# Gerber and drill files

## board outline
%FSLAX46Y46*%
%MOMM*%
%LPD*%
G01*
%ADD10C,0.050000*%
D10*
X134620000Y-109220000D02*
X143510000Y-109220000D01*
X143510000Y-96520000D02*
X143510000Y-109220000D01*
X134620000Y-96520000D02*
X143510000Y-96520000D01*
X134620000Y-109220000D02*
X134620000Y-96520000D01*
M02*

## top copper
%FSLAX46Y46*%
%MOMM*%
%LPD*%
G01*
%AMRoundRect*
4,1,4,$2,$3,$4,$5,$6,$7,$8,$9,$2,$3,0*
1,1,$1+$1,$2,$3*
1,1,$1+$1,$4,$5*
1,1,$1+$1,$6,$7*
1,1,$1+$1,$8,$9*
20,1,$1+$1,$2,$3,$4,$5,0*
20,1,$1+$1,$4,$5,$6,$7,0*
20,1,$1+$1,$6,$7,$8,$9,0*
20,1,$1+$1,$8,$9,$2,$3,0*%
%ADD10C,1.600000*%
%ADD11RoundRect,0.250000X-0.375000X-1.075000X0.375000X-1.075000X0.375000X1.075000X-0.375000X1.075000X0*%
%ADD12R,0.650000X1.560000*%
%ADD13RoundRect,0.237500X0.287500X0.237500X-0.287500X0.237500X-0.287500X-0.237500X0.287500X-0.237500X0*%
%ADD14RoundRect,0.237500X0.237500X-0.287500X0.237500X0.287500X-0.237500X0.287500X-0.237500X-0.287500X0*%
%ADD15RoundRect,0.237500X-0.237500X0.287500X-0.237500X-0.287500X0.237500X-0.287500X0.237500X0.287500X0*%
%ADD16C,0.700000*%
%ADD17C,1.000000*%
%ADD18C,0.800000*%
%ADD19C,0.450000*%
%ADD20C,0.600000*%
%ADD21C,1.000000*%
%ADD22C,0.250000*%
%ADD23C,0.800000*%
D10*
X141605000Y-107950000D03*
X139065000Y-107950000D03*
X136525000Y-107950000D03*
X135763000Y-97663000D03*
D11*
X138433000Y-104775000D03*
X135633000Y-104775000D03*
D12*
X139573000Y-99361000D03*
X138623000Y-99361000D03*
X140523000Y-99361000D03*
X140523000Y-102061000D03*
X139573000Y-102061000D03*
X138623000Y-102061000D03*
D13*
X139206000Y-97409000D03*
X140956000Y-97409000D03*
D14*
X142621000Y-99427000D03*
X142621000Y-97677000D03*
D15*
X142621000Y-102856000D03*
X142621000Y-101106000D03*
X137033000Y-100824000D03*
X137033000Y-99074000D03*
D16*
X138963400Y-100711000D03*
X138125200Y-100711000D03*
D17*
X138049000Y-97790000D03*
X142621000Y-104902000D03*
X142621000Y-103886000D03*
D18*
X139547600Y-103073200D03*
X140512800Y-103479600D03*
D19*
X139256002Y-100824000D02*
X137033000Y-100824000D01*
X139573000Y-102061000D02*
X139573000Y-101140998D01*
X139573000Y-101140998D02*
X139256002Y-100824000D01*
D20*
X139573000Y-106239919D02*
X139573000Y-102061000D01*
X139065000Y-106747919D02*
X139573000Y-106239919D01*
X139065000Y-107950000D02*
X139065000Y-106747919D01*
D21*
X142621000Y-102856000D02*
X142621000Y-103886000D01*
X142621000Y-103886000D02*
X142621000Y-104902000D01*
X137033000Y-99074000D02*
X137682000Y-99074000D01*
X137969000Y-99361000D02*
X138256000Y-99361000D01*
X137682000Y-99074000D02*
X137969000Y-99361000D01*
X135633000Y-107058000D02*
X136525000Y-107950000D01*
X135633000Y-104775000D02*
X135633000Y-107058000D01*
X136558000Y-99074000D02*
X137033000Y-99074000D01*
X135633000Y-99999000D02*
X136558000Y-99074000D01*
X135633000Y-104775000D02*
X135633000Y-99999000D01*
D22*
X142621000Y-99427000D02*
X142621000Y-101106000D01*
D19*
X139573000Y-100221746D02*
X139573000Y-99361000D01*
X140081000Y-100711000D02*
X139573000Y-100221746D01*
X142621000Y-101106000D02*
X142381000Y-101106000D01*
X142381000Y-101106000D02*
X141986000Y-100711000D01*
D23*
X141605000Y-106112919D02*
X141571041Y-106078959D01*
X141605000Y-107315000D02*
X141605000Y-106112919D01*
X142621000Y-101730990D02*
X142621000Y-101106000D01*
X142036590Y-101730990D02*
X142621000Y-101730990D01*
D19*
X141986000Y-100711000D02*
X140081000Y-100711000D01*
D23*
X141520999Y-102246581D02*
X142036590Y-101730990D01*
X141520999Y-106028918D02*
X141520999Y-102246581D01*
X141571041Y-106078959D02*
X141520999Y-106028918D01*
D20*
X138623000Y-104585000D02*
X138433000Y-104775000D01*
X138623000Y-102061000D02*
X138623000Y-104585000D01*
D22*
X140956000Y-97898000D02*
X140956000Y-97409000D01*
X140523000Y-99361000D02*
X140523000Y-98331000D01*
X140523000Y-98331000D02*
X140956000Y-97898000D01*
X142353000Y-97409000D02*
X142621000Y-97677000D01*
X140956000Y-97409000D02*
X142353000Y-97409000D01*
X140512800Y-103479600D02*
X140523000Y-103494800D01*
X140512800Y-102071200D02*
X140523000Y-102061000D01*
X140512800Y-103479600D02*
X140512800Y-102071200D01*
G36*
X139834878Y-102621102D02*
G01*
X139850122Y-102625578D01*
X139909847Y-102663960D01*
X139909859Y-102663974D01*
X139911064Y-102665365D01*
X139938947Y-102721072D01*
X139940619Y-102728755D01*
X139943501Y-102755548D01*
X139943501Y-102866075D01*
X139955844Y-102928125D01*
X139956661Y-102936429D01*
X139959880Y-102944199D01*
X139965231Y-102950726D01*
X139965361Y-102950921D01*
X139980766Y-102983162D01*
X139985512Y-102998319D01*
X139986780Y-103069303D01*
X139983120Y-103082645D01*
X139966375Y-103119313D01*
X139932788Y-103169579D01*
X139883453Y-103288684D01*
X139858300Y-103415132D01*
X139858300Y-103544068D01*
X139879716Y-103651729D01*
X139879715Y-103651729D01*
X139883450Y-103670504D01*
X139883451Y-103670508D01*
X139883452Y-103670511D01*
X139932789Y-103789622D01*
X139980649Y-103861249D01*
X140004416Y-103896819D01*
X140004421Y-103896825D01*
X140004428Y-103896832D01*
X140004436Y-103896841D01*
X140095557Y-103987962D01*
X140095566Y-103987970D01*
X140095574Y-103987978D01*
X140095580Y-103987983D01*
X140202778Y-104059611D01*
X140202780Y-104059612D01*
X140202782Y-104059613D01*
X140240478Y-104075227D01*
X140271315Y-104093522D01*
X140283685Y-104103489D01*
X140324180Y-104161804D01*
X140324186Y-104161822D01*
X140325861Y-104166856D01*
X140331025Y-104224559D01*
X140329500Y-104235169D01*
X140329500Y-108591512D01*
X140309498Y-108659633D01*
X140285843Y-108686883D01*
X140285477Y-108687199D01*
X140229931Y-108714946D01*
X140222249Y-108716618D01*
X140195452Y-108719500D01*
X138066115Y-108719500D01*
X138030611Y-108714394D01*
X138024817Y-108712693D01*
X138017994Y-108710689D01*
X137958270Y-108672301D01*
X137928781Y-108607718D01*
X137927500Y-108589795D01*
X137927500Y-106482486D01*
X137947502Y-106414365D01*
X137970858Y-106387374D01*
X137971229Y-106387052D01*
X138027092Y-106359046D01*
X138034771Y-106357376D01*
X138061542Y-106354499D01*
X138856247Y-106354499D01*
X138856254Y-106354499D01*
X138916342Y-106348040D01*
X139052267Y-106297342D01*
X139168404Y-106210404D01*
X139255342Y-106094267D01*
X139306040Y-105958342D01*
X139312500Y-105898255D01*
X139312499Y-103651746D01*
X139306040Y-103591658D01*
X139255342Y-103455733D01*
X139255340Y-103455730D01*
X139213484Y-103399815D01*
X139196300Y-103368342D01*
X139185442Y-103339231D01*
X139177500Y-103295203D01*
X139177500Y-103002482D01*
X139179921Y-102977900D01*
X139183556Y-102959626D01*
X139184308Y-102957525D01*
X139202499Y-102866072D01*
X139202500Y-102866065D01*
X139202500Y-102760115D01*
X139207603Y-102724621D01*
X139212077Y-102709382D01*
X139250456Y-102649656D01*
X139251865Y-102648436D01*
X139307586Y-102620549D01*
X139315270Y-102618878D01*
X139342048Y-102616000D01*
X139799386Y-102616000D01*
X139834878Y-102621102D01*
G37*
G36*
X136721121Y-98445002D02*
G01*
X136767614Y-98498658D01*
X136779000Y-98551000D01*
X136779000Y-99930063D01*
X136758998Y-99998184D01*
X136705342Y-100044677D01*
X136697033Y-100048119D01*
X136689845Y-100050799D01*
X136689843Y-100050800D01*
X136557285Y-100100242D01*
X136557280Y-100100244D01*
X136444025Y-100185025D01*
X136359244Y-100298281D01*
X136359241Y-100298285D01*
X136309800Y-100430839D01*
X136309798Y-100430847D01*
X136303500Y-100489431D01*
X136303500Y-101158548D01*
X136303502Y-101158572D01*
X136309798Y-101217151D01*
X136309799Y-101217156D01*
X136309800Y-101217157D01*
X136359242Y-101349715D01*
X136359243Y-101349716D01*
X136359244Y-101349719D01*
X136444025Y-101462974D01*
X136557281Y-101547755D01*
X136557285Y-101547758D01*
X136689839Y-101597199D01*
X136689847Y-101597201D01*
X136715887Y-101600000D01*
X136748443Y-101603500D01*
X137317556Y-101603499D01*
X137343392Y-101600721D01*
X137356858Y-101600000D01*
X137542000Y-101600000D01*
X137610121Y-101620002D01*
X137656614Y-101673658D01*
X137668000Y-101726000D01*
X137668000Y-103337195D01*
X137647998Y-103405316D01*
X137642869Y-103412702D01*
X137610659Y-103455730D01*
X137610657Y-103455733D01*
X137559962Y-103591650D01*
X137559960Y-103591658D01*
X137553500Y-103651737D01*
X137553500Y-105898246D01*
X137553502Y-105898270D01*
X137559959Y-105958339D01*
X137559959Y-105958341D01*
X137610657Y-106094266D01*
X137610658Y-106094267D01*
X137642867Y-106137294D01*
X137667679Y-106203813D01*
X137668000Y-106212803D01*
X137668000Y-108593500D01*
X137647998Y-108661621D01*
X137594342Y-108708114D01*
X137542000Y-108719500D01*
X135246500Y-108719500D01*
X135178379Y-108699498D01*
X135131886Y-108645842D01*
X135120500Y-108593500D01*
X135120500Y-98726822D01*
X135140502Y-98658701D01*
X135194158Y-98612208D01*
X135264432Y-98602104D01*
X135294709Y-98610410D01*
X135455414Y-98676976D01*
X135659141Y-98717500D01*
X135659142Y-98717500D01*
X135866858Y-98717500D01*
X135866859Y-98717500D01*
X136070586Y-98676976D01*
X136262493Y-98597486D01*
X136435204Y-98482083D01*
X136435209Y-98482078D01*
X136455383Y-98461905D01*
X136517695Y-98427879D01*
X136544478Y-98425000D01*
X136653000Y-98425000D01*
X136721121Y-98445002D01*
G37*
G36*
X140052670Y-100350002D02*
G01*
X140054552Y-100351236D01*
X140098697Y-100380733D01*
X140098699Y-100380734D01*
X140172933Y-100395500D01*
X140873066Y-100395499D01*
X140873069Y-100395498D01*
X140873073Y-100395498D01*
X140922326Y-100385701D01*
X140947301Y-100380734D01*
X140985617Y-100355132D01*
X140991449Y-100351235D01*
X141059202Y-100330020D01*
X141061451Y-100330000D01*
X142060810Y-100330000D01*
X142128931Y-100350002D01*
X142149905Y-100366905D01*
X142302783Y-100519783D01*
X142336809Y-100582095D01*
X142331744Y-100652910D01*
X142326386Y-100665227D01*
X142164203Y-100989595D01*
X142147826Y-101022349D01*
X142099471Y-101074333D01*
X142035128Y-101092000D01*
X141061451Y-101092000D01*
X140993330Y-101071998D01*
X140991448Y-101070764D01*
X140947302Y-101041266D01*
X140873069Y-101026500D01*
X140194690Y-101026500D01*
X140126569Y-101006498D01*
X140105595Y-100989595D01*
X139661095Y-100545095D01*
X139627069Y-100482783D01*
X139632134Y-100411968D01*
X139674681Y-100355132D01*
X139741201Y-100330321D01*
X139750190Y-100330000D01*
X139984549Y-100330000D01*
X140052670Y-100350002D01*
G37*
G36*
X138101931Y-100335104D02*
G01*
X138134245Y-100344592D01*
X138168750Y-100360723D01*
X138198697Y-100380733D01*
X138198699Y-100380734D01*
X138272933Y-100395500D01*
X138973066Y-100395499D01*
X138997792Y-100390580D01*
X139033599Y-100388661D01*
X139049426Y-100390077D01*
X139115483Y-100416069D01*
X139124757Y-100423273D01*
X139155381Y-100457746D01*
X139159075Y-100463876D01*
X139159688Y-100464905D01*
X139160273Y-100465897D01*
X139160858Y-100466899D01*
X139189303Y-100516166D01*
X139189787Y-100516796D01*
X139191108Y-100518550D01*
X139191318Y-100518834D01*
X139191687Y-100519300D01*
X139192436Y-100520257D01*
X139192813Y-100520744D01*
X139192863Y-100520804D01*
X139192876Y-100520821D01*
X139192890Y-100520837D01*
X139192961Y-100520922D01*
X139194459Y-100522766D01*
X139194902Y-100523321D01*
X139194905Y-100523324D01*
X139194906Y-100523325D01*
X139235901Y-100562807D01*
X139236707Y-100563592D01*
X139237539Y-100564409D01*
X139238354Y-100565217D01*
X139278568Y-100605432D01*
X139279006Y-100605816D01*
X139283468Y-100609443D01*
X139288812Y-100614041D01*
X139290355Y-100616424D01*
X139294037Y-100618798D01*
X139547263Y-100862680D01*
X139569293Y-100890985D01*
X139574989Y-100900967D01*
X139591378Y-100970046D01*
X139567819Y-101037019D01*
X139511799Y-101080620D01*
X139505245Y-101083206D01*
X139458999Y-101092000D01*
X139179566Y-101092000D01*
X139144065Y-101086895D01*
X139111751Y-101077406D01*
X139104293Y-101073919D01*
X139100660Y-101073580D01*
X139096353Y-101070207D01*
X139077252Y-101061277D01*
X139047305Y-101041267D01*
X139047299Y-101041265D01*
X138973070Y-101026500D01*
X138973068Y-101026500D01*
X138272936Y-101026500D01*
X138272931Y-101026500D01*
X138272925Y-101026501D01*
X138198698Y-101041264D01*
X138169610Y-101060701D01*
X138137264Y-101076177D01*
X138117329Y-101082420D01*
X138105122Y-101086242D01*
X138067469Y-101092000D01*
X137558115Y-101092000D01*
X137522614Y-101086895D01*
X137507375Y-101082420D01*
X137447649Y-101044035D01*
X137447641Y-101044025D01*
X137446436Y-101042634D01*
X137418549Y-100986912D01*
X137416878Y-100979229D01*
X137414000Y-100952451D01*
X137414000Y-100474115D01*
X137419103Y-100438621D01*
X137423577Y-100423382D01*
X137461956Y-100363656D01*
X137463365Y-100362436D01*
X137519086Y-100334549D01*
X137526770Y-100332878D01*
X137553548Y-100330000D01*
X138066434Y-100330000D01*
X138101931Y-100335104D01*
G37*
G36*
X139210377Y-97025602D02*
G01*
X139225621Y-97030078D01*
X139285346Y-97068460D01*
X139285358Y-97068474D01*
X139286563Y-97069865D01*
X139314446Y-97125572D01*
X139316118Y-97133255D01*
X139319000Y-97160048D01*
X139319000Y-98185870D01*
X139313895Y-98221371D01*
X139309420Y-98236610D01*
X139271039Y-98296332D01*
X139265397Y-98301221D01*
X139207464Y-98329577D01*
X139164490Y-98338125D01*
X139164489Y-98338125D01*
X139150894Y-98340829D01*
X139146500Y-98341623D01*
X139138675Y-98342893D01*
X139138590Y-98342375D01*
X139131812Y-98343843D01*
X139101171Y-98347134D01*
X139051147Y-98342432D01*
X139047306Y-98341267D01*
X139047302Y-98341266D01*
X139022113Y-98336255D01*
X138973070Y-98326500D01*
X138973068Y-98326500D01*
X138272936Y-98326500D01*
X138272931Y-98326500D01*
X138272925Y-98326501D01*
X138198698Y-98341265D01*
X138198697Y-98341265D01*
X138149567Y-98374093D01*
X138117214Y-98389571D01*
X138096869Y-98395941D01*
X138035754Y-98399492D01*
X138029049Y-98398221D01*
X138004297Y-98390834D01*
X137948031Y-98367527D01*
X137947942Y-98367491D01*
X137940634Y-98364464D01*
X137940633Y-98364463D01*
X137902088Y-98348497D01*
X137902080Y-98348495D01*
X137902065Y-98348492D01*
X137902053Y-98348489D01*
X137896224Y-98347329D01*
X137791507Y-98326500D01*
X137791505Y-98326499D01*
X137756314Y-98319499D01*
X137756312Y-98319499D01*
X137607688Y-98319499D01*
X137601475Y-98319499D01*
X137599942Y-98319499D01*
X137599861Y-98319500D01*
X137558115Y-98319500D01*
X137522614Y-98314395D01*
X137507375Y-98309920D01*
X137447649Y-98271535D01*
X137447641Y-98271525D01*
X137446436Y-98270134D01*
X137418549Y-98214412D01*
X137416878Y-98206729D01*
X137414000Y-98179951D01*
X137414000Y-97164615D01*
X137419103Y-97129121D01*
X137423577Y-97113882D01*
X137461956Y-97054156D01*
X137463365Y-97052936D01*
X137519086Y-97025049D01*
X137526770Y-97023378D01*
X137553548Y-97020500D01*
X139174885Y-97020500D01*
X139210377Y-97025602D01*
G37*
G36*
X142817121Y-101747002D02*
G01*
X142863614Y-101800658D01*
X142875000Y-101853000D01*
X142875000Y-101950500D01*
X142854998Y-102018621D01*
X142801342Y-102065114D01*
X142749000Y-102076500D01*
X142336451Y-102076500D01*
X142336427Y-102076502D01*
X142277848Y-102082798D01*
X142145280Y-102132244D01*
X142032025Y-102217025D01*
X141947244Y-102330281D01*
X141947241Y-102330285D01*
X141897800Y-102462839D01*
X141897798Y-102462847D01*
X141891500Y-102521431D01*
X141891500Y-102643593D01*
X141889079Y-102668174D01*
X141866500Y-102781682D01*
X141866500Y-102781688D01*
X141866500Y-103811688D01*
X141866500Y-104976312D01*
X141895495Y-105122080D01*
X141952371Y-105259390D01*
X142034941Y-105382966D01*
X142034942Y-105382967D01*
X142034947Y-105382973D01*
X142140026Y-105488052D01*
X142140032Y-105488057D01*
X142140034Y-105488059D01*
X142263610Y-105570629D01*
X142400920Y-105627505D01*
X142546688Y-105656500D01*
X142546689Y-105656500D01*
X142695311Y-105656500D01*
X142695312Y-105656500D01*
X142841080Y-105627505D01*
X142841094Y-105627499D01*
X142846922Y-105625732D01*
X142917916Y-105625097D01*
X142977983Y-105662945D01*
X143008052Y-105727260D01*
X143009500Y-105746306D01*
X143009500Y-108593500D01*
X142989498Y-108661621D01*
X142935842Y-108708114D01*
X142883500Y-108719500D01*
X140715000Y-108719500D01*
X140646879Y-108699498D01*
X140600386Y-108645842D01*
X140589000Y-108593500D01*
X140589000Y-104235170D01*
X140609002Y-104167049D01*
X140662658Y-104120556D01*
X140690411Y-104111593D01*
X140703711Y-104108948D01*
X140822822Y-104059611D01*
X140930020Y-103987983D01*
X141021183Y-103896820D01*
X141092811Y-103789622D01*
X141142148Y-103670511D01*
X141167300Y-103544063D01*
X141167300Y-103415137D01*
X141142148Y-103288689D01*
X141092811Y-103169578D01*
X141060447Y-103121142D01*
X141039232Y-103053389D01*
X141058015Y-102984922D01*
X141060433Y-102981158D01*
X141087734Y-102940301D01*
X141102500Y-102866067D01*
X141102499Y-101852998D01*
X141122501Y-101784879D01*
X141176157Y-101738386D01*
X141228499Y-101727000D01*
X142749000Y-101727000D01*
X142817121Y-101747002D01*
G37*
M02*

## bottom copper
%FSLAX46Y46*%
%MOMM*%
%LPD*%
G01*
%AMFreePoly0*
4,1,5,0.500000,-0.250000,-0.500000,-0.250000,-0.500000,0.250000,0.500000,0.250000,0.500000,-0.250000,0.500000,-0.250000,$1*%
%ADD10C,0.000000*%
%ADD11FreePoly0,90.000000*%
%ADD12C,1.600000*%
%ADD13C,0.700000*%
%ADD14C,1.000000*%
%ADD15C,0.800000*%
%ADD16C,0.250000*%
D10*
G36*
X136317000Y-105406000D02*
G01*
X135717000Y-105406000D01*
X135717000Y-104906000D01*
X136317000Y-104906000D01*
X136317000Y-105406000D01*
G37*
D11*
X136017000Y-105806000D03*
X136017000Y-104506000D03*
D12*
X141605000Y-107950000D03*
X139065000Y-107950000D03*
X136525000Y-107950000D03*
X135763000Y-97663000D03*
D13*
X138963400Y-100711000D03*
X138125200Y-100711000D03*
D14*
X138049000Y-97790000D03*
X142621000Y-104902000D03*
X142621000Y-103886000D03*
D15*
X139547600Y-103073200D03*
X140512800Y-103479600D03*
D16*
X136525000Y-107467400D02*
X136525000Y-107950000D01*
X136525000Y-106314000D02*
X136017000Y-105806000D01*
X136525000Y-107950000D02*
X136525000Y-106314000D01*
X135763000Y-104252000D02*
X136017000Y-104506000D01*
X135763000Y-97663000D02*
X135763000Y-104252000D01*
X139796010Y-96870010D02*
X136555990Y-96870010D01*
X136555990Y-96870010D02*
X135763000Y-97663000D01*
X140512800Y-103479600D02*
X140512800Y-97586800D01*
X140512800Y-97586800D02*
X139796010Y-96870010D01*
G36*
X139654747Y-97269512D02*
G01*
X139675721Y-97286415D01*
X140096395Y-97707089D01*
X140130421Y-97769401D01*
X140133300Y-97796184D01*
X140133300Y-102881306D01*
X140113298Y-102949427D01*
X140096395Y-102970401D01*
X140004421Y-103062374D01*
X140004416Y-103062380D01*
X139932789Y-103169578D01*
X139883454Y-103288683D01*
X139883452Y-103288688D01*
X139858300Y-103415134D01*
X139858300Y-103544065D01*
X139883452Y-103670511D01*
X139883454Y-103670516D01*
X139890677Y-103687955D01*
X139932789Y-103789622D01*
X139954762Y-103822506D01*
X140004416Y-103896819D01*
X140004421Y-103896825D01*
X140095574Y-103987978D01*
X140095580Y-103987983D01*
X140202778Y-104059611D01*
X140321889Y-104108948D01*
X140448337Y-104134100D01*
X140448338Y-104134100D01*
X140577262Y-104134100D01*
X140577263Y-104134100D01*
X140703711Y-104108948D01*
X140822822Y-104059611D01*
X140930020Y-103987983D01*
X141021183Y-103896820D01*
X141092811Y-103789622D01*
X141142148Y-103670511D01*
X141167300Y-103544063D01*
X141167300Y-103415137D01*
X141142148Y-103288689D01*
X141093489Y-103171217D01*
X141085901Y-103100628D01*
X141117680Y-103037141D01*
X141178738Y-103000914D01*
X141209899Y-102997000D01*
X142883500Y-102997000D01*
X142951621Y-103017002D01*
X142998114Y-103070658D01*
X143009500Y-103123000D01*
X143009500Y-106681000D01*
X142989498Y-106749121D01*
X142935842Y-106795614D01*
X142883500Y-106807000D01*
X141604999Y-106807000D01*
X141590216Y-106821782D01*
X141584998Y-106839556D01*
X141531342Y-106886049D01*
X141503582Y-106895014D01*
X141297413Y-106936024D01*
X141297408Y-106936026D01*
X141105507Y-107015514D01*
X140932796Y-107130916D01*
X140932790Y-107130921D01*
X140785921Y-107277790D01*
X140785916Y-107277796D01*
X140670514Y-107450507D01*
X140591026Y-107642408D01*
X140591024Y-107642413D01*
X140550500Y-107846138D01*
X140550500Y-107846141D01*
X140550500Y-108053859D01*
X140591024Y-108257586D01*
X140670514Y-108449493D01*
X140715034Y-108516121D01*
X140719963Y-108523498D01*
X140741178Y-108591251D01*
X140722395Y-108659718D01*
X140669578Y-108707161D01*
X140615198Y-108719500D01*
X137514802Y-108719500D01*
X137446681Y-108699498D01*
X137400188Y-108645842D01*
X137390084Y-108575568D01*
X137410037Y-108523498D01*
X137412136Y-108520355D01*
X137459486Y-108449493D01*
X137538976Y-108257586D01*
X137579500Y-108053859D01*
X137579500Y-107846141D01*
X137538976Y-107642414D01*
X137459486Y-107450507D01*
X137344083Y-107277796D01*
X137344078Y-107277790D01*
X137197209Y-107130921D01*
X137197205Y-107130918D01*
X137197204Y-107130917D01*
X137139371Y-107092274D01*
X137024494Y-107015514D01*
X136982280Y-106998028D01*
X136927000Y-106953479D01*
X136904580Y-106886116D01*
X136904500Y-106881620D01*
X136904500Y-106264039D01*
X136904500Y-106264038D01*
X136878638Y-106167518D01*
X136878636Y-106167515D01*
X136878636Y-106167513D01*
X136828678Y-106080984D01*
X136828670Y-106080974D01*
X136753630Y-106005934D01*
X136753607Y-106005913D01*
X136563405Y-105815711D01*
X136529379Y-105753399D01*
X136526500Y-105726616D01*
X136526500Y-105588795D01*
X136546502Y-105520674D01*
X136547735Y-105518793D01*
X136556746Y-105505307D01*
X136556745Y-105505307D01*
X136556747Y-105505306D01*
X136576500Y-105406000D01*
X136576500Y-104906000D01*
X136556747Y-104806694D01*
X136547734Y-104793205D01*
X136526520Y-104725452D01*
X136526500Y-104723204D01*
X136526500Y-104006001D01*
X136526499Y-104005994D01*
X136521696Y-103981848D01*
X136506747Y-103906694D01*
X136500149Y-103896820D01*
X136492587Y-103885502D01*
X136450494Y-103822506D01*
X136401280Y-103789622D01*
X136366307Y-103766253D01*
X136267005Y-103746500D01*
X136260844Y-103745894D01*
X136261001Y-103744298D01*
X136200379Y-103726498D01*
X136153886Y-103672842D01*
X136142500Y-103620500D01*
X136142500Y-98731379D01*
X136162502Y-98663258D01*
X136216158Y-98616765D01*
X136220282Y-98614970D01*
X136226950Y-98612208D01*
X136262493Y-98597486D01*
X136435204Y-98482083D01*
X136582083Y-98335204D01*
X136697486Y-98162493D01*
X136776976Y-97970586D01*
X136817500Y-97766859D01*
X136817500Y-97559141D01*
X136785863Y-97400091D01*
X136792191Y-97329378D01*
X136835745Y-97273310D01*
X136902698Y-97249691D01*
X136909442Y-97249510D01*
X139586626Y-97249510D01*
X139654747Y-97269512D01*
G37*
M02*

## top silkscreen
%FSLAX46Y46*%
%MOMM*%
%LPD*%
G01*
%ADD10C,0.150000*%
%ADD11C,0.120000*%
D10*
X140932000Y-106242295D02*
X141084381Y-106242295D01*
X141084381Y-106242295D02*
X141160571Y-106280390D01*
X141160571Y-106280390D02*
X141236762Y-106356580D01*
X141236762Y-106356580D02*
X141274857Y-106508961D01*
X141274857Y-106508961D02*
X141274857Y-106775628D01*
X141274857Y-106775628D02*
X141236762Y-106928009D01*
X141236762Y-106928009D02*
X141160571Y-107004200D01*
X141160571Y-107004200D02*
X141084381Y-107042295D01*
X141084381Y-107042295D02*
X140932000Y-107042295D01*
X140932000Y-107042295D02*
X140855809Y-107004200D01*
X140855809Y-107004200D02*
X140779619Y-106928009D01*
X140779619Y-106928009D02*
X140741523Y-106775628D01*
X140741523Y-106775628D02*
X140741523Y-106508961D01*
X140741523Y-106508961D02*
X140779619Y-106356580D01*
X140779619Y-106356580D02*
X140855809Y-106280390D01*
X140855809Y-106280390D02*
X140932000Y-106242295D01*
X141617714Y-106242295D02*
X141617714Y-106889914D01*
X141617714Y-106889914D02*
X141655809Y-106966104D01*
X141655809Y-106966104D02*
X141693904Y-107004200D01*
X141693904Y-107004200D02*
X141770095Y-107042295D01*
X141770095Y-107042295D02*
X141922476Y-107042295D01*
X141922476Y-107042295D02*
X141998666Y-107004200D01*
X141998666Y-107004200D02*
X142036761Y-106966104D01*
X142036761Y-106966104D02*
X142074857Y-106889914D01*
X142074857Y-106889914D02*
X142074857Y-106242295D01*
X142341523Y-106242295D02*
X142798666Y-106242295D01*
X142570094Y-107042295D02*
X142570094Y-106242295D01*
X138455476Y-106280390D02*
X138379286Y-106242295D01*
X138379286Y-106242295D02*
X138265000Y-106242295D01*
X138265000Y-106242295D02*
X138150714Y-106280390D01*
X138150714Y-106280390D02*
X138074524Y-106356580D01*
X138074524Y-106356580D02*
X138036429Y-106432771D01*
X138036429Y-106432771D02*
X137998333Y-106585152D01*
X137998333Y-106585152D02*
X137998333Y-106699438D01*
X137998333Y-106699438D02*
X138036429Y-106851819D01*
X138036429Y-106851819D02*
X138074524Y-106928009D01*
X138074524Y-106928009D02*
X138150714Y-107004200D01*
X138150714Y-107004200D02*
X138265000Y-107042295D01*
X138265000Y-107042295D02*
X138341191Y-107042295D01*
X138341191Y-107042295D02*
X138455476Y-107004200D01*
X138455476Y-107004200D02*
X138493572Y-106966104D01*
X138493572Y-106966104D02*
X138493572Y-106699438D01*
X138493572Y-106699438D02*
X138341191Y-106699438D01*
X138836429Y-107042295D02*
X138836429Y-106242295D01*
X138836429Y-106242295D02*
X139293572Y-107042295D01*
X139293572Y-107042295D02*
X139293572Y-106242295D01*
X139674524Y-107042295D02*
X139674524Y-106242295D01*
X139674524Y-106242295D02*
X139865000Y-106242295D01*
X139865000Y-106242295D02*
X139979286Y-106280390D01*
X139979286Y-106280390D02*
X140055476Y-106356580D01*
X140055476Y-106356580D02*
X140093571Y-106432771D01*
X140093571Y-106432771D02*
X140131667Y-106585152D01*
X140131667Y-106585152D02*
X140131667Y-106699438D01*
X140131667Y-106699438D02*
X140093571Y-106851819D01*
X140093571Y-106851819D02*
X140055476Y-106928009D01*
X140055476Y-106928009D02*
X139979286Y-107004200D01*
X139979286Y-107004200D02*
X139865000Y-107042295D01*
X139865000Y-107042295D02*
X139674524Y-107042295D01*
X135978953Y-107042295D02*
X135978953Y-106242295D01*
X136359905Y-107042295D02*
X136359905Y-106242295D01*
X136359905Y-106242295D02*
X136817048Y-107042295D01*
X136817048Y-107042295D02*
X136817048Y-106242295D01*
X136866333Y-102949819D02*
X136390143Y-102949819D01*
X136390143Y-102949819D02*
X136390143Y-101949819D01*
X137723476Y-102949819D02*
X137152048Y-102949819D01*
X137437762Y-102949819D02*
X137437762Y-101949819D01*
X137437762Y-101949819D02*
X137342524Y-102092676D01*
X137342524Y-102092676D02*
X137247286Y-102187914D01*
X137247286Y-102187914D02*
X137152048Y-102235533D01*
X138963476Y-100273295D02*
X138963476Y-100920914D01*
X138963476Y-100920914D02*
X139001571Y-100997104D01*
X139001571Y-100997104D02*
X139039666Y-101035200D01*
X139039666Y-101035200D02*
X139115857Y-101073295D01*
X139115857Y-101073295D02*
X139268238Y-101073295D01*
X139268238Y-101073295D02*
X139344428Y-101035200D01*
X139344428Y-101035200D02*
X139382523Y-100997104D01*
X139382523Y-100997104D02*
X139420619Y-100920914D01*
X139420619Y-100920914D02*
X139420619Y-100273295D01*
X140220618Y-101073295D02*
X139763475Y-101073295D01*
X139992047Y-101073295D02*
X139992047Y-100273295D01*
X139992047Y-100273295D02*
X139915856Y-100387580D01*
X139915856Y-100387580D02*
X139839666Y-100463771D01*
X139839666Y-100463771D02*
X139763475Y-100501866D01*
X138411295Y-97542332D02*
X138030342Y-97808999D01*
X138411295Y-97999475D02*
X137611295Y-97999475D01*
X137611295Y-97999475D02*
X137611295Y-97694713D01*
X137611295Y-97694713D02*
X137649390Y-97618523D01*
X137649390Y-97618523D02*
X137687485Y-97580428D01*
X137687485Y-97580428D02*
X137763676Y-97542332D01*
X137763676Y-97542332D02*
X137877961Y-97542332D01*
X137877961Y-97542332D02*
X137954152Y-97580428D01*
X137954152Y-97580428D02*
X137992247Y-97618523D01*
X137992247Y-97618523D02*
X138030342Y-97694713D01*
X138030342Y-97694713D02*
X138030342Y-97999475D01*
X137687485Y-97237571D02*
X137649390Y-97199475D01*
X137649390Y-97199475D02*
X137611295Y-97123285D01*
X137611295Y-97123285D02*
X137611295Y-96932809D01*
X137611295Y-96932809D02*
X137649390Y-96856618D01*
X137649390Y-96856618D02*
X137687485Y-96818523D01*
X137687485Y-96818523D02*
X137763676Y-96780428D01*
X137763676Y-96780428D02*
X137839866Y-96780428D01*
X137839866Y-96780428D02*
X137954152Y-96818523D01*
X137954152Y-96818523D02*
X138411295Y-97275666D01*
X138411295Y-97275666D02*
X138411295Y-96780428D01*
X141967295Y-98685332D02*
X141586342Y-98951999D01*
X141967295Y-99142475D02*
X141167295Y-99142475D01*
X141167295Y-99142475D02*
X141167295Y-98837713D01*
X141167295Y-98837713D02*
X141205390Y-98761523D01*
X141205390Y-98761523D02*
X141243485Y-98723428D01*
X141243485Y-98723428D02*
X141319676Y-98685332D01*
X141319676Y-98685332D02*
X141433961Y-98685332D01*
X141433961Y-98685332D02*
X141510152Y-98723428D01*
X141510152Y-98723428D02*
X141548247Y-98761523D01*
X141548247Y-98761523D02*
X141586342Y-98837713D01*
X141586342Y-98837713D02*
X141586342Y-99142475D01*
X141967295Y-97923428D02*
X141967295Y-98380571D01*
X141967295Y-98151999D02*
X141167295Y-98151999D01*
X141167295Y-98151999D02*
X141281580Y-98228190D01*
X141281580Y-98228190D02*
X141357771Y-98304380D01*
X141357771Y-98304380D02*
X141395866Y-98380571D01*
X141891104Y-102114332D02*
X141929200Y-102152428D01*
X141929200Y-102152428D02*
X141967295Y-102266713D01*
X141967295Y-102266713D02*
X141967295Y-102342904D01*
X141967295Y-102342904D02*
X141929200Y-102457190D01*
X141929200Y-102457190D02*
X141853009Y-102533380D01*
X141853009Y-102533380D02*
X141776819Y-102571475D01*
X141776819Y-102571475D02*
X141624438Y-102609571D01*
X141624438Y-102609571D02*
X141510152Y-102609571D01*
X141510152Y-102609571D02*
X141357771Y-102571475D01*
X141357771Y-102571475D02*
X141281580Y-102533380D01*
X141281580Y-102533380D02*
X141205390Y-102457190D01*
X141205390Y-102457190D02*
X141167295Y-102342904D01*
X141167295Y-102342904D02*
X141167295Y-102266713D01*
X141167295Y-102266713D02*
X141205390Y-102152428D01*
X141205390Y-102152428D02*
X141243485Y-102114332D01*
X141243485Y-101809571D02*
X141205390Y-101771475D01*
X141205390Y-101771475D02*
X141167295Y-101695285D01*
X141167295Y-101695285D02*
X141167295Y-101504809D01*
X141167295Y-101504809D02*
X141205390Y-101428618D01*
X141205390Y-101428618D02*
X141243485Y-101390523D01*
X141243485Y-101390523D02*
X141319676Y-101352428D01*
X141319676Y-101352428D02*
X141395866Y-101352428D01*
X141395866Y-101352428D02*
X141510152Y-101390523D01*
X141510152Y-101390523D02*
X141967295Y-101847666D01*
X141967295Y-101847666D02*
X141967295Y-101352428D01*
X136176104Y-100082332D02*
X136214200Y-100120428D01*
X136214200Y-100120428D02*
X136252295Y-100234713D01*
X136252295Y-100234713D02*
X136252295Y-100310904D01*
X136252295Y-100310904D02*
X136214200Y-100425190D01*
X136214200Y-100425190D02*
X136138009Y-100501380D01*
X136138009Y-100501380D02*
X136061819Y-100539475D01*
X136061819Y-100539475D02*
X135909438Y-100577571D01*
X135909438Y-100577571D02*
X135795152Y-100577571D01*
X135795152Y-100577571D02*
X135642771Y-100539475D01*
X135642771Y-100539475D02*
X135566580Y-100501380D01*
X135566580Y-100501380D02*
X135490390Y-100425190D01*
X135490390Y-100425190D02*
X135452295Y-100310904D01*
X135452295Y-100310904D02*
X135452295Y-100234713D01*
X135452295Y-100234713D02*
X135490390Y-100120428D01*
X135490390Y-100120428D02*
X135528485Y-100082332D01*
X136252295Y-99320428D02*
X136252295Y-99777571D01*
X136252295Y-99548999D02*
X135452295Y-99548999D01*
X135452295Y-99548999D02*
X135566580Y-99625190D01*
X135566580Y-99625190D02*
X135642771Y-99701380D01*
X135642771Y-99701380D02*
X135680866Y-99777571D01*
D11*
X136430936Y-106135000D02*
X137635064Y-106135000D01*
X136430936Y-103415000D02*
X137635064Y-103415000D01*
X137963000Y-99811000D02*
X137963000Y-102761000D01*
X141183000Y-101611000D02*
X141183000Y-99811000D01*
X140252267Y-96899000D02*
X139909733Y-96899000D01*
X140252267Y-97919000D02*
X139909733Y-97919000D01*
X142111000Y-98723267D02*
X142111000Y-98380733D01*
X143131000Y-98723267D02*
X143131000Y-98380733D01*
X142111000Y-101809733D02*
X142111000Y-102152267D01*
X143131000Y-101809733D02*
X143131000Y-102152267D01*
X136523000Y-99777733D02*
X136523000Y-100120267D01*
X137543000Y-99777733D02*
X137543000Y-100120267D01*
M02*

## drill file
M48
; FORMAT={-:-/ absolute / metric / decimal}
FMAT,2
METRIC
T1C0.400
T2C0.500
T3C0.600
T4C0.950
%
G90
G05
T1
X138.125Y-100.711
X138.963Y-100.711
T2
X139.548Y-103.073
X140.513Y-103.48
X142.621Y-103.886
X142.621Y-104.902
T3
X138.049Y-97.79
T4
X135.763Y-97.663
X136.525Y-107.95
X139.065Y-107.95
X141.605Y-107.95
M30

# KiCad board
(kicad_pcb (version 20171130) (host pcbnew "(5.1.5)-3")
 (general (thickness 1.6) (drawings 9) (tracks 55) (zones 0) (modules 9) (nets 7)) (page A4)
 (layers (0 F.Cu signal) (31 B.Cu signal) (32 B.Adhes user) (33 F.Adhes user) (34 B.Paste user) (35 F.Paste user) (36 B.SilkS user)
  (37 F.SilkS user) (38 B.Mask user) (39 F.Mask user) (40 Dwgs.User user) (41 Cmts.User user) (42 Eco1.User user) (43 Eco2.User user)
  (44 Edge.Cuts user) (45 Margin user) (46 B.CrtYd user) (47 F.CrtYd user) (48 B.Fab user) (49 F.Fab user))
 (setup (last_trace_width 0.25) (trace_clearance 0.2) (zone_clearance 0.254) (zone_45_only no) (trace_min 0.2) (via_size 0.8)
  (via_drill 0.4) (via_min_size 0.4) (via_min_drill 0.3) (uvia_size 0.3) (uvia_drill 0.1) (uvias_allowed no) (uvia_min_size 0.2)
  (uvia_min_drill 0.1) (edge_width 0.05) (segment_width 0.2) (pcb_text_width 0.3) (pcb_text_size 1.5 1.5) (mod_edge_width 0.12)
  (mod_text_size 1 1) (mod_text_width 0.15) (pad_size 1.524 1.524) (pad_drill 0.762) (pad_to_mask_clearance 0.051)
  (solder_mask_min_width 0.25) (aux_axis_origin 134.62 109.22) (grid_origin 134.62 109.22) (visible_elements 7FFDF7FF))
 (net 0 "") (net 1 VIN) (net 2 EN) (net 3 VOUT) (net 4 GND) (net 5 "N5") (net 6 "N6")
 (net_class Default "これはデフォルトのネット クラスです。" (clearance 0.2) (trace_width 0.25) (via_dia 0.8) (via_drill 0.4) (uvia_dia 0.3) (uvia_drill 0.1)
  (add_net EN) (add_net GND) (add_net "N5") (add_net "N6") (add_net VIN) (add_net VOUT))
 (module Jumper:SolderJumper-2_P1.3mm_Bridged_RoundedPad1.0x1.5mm (layer B.Cu) (at 136.017 105.156 90)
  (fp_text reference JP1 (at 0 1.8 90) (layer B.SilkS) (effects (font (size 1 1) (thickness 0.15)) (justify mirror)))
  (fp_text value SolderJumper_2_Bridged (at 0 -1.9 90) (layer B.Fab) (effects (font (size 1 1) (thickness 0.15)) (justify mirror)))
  (fp_poly (pts (xy 0.25 0.3) (xy -0.25 0.3) (xy -0.25 -0.3) (xy 0.25 -0.3)) (layer B.Cu) (width 0))
  (pad 1 smd custom (at -0.65 0 90) (size 1 0.5) (layers B.Cu B.Mask) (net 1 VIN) (zone_connect 2)
   (options (clearance outline) (anchor rect)) (primitives))
  (pad 2 smd custom (at 0.65 0 90) (size 1 0.5) (layers B.Cu B.Mask) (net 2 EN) (zone_connect 2) (options (clearance outline) (anchor rect))
   (primitives)))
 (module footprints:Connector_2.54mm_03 (layer F.Cu) (at 136.525 107.95 90)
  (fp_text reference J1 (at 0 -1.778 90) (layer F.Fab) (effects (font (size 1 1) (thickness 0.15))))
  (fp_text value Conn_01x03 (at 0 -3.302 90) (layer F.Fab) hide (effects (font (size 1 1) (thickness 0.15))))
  (pad 3 thru_hole circle (at 0 5.08 90) (size 1.6 1.6) (drill 0.95) (layers *.Cu *.Mask) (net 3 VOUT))
  (pad 2 thru_hole circle (at 0 2.54 90) (size 1.6 1.6) (drill 0.95) (layers *.Cu *.Mask) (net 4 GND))
  (pad 1 thru_hole circle (at 0 0 90) (size 1.6 1.6) (drill 0.95) (layers *.Cu *.Mask) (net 1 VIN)))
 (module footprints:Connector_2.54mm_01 (layer F.Cu) (at 135.763 97.663)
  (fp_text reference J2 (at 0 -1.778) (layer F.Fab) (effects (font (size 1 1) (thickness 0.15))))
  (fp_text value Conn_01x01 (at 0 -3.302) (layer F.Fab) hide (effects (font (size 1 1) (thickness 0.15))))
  (pad 1 thru_hole circle (at 0 0) (size 1.6 1.6) (drill 0.95) (layers *.Cu *.Mask) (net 2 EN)))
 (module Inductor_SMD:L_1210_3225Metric (layer F.Cu) (at 137.033 104.775)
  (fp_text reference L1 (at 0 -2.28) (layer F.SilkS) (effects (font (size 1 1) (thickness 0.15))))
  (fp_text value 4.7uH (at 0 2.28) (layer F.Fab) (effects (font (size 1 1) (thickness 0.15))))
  (fp_line (start -0.602064 1.36) (end 0.602064 1.36) (layer F.SilkS) (width 0.12))
  (fp_line (start -0.602064 -1.36) (end 0.602064 -1.36) (layer F.SilkS) (width 0.12))
  (pad 2 smd roundrect (at 1.4 0) (size 1.25 2.65) (layers F.Cu F.Paste F.Mask) (roundrect_rratio 0.2) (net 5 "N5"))
  (pad 1 smd roundrect (at -1.4 0) (size 1.25 2.65) (layers F.Cu F.Paste F.Mask) (roundrect_rratio 0.2) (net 1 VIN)))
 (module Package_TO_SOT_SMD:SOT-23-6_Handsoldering (layer F.Cu) (at 139.573 100.711 90)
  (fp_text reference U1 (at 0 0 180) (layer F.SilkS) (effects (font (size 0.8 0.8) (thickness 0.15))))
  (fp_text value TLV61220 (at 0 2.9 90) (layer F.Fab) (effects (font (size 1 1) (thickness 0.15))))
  (fp_line (start 0.9 -1.61) (end -2.05 -1.61) (layer F.SilkS) (width 0.12))
  (fp_line (start -0.9 1.61) (end 0.9 1.61) (layer F.SilkS) (width 0.12))
  (pad 5 smd rect (at 1.35 0 90) (size 1.56 0.65) (layers F.Cu F.Paste F.Mask) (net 3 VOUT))
  (pad 6 smd rect (at 1.35 -0.95 90) (size 1.56 0.65) (layers F.Cu F.Paste F.Mask) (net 1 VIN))
  (pad 4 smd rect (at 1.35 0.95 90) (size 1.56 0.65) (layers F.Cu F.Paste F.Mask) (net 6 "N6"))
  (pad 3 smd rect (at -1.35 0.95 90) (size 1.56 0.65) (layers F.Cu F.Paste F.Mask) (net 2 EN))
  (pad 2 smd rect (at -1.35 0 90) (size 1.56 0.65) (layers F.Cu F.Paste F.Mask) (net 4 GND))
  (pad 1 smd rect (at -1.35 -0.95 90) (size 1.56 0.65) (layers F.Cu F.Paste F.Mask) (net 5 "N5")))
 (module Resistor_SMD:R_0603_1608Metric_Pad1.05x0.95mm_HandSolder (layer F.Cu) (at 140.081 97.409 180)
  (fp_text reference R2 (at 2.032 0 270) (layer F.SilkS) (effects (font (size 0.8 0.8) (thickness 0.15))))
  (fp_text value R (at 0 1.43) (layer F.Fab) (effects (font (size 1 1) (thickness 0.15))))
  (fp_line (start -0.171267 0.51) (end 0.171267 0.51) (layer F.SilkS) (width 0.12))
  (fp_line (start -0.171267 -0.51) (end 0.171267 -0.51) (layer F.SilkS) (width 0.12))
  (pad 2 smd roundrect (at 0.875 0 180) (size 1.05 0.95) (layers F.Cu F.Paste F.Mask) (roundrect_rratio 0.25) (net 4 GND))
  (pad 1 smd roundrect (at -0.875 0 180) (size 1.05 0.95) (layers F.Cu F.Paste F.Mask) (roundrect_rratio 0.25) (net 6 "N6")))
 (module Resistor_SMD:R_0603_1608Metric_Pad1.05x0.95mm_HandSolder (layer F.Cu) (at 142.621 98.552 90)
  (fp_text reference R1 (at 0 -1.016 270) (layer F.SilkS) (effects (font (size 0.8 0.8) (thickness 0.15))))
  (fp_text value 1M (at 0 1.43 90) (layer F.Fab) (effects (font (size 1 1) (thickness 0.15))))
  (fp_line (start -0.171267 -0.51) (end 0.171267 -0.51) (layer F.SilkS) (width 0.12))
  (fp_line (start -0.171267 0.51) (end 0.171267 0.51) (layer F.SilkS) (width 0.12))
  (pad 1 smd roundrect (at -0.875 0 90) (size 1.05 0.95) (layers F.Cu F.Paste F.Mask) (roundrect_rratio 0.25) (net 3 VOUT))
  (pad 2 smd roundrect (at 0.875 0 90) (size 1.05 0.95) (layers F.Cu F.Paste F.Mask) (roundrect_rratio 0.25) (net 6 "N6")))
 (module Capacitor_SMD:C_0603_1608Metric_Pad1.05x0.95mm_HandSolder (layer F.Cu) (at 142.621 101.981 270)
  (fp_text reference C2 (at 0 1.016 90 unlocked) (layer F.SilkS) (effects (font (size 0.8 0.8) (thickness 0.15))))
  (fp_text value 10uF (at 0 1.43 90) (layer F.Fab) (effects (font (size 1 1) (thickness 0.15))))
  (fp_line (start -0.171267 0.51) (end 0.171267 0.51) (layer F.SilkS) (width 0.12))
  (fp_line (start -0.171267 -0.51) (end 0.171267 -0.51) (layer F.SilkS) (width 0.12))
  (pad 2 smd roundrect (at 0.875 0 270) (size 1.05 0.95) (layers F.Cu F.Paste F.Mask) (roundrect_rratio 0.25) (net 4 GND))
  (pad 1 smd roundrect (at -0.875 0 270) (size 1.05 0.95) (layers F.Cu F.Paste F.Mask) (roundrect_rratio 0.25) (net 3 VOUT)))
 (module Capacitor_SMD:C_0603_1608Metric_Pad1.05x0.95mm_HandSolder (layer F.Cu) (at 137.033 99.949 270)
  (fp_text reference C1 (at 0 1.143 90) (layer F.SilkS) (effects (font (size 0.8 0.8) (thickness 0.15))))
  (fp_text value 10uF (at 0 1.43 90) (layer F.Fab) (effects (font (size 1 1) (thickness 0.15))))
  (fp_line (start -0.171267 0.51) (end 0.171267 0.51) (layer F.SilkS) (width 0.12))
  (fp_line (start -0.171267 -0.51) (end 0.171267 -0.51) (layer F.SilkS) (width 0.12))
  (pad 2 smd roundrect (at 0.875 0 270) (size 1.05 0.95) (layers F.Cu F.Paste F.Mask) (roundrect_rratio 0.25) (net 4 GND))
  (pad 1 smd roundrect (at -0.875 0 270) (size 1.05 0.95) (layers F.Cu F.Paste F.Mask) (roundrect_rratio 0.25) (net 1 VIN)))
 (gr_line (start 134.62 109.22) (end 143.51 109.22) (layer Edge.Cuts) (width 0.05))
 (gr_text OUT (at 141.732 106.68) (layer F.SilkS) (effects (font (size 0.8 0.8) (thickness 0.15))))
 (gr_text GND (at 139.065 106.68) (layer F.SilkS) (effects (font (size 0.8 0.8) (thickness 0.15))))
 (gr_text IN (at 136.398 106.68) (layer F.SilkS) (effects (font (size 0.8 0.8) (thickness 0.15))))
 (gr_line (start 143.51 96.52) (end 143.51 109.22) (layer Edge.Cuts) (width 0.05))
 (gr_line (start 134.62 96.52) (end 143.51 96.52) (layer Edge.Cuts) (width 0.05))
 (gr_line (start 134.62 109.22) (end 134.62 96.52) (layer Edge.Cuts) (width 0.05))
 (via (at 138.9634 100.711) (size 0.7) (drill 0.4) (layers F.Cu B.Cu) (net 4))
 (via (at 138.1252 100.711) (size 0.7) (drill 0.4) (layers F.Cu B.Cu) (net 4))
 (via (at 138.049 97.79) (size 1) (drill 0.6) (layers F.Cu B.Cu) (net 4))
 (segment (start 139.256002 100.824) (end 137.033 100.824) (width 0.45) (layer F.Cu) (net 4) (status 20))
 (segment (start 139.573 102.061) (end 139.573 101.140998) (width 0.45) (layer F.Cu) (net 4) (status 10))
 (segment (start 139.573 101.140998) (end 139.256002 100.824) (width 0.45) (layer F.Cu) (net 4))
 (via (at 142.621 104.902) (size 1) (drill 0.5) (layers F.Cu B.Cu) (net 4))
 (via (at 142.621 103.886) (size 1) (drill 0.5) (layers F.Cu B.Cu) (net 4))
 (segment (start 139.573 106.239919) (end 139.573 102.061) (width 0.6) (layer F.Cu) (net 4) (status 20))
 (segment (start 139.065 106.747919) (end 139.573 106.239919) (width 0.6) (layer F.Cu) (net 4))
 (segment (start 139.065 107.95) (end 139.065 106.747919) (width 0.6) (layer F.Cu) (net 4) (status 10))
 (segment (start 142.621 102.856) (end 142.621 103.886) (width 1) (layer F.Cu) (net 4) (status 10))
 (segment (start 142.621 103.886) (end 142.621 104.902) (width 1) (layer F.Cu) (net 4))
 (via (at 139.5476 103.0732) (size 0.8) (drill 0.5) (layers F.Cu B.Cu) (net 4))
 (segment (start 137.033 99.074) (end 137.682 99.074) (width 1) (layer F.Cu) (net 1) (status 10))
 (segment (start 137.969 99.361) (end 138.256 99.361) (width 1) (layer F.Cu) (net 1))
 (segment (start 137.682 99.074) (end 137.969 99.361) (width 1) (layer F.Cu) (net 1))
 (segment (start 135.633 107.058) (end 136.525 107.95) (width 1) (layer F.Cu) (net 1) (status 20))
 (segment (start 135.633 104.775) (end 135.633 107.058) (width 1) (layer F.Cu) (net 1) (status 10))
 (segment (start 136.558 99.074) (end 137.033 99.074) (width 1) (layer F.Cu) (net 1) (status 30))
 (segment (start 135.633 99.999) (end 136.558 99.074) (width 1) (layer F.Cu) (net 1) (status 20))
 (segment (start 135.633 104.775) (end 135.633 99.999) (width 1) (layer F.Cu) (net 1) (status 10))
 (segment (start 136.525 107.4674) (end 136.525 107.95) (width 0.25) (layer B.Cu) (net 1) (status 30))
 (segment (start 136.525 106.314) (end 136.017 105.806) (width 0.25) (layer B.Cu) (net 1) (status 20))
 (segment (start 136.525 107.95) (end 136.525 106.314) (width 0.25) (layer B.Cu) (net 1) (status 10))
 (segment (start 142.621 99.427) (end 142.621 101.106) (width 0.25) (layer F.Cu) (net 3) (status 30))
 (segment (start 139.573 100.221746) (end 139.573 99.361) (width 0.45) (layer F.Cu) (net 3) (status 20))
 (segment (start 140.081 100.711) (end 139.573 100.221746) (width 0.45) (layer F.Cu) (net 3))
 (segment (start 142.621 101.106) (end 142.381 101.106) (width 0.45) (layer F.Cu) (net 3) (status 30))
 (segment (start 142.381 101.106) (end 141.986 100.711) (width 0.45) (layer F.Cu) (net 3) (status 10))
 (segment (start 141.605 106.112919) (end 141.571041 106.078959) (width 0.8) (layer F.Cu) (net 3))
 (segment (start 141.605 107.315) (end 141.605 106.112919) (width 0.8) (layer F.Cu) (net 3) (status 10))
 (segment (start 142.621 101.73099) (end 142.621 101.106) (width 0.8) (layer F.Cu) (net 3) (status 20))
 (segment (start 142.03659 101.73099) (end 142.621 101.73099) (width 0.8) (layer F.Cu) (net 3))
 (segment (start 141.986 100.711) (end 140.081 100.711) (width 0.45) (layer F.Cu) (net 3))
 (segment (start 141.520999 102.246581) (end 142.03659 101.73099) (width 0.8) (layer F.Cu) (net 3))
 (segment (start 141.520999 106.028918) (end 141.520999 102.246581) (width 0.8) (layer F.Cu) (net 3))
 (segment (start 141.571041 106.078959) (end 141.520999 106.028918) (width 0.8) (layer F.Cu) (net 3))
 (segment (start 138.623 104.585) (end 138.433 104.775) (width 0.6) (layer F.Cu) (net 5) (status 30))
 (segment (start 138.623 102.061) (end 138.623 104.585) (width 0.6) (layer F.Cu) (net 5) (status 30))
 (segment (start 140.956 97.898) (end 140.956 97.409) (width 0.25) (layer F.Cu) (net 6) (status 20))
 (segment (start 140.523 99.361) (end 140.523 98.331) (width 0.25) (layer F.Cu) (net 6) (status 10))
 (segment (start 140.523 98.331) (end 140.956 97.898) (width 0.25) (layer F.Cu) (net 6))
 (segment (start 142.353 97.409) (end 142.621 97.677) (width 0.25) (layer F.Cu) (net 6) (status 30))
 (segment (start 140.956 97.409) (end 142.353 97.409) (width 0.25) (layer F.Cu) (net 6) (status 30))
 (via (at 140.5128 103.4796) (size 0.8) (drill 0.5) (layers F.Cu B.Cu) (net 2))
 (segment (start 140.5128 103.4796) (end 140.523 103.4948) (width 0.25) (layer F.Cu) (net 2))
 (segment (start 140.5128 102.0712) (end 140.523 102.061) (width 0.25) (layer F.Cu) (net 2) (status 30))
 (segment (start 140.5128 103.4796) (end 140.5128 102.0712) (width 0.25) (layer F.Cu) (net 2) (status 20))
 (segment (start 135.763 104.252) (end 136.017 104.506) (width 0.25) (layer B.Cu) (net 2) (status 30))
 (segment (start 135.763 97.663) (end 135.763 104.252) (width 0.25) (layer B.Cu) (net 2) (status 30))
 (segment (start 139.79601 96.87001) (end 136.55599 96.87001) (width 0.25) (layer B.Cu) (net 2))
 (segment (start 136.55599 96.87001) (end 135.763 97.663) (width 0.25) (layer B.Cu) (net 2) (status 20))
 (segment (start 140.5128 103.4796) (end 140.5128 97.5868) (width 0.25) (layer B.Cu) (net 2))
 (segment (start 140.5128 97.5868) (end 139.79601 96.87001) (width 0.25) (layer B.Cu) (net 2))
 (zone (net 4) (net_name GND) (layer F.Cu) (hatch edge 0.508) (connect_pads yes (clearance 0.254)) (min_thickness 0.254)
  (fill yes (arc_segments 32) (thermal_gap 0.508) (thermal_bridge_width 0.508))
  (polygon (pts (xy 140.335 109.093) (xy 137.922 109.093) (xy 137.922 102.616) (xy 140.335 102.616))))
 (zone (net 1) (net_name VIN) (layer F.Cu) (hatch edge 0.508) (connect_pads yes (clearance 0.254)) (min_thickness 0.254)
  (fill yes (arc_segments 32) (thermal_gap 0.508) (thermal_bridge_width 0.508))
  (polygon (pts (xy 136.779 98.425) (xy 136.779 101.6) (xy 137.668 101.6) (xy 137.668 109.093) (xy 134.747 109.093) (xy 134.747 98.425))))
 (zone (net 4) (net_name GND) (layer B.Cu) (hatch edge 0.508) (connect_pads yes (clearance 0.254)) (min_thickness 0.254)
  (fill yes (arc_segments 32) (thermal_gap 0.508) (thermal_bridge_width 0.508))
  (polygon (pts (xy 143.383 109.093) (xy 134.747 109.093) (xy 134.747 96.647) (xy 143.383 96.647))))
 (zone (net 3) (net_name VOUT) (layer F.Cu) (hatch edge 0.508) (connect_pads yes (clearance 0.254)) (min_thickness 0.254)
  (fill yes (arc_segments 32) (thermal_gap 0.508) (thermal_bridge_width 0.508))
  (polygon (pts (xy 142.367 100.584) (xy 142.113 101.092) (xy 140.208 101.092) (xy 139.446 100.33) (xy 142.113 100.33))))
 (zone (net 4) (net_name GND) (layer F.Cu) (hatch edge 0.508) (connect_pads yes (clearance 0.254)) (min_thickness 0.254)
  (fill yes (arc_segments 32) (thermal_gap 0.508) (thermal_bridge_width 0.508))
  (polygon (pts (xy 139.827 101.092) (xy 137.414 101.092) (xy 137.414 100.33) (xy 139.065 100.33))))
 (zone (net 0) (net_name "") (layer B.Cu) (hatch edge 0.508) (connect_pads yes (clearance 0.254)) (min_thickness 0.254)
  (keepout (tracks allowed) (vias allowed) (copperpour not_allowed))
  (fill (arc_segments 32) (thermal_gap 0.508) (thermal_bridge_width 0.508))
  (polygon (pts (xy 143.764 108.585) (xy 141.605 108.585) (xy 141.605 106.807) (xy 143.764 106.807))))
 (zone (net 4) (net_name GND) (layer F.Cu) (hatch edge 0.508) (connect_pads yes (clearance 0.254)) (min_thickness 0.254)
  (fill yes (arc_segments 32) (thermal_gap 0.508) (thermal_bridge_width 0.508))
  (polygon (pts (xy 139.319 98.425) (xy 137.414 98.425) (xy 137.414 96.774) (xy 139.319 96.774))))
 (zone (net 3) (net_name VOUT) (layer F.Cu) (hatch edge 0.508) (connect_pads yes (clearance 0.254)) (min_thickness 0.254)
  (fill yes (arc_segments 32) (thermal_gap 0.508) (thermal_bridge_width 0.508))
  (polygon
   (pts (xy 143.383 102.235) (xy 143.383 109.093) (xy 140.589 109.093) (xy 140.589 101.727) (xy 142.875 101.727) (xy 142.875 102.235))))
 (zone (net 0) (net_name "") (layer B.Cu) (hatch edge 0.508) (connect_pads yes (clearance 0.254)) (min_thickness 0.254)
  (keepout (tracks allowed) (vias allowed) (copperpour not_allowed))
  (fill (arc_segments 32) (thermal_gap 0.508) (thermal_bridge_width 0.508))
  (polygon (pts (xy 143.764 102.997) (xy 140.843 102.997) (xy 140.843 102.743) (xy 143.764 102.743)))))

